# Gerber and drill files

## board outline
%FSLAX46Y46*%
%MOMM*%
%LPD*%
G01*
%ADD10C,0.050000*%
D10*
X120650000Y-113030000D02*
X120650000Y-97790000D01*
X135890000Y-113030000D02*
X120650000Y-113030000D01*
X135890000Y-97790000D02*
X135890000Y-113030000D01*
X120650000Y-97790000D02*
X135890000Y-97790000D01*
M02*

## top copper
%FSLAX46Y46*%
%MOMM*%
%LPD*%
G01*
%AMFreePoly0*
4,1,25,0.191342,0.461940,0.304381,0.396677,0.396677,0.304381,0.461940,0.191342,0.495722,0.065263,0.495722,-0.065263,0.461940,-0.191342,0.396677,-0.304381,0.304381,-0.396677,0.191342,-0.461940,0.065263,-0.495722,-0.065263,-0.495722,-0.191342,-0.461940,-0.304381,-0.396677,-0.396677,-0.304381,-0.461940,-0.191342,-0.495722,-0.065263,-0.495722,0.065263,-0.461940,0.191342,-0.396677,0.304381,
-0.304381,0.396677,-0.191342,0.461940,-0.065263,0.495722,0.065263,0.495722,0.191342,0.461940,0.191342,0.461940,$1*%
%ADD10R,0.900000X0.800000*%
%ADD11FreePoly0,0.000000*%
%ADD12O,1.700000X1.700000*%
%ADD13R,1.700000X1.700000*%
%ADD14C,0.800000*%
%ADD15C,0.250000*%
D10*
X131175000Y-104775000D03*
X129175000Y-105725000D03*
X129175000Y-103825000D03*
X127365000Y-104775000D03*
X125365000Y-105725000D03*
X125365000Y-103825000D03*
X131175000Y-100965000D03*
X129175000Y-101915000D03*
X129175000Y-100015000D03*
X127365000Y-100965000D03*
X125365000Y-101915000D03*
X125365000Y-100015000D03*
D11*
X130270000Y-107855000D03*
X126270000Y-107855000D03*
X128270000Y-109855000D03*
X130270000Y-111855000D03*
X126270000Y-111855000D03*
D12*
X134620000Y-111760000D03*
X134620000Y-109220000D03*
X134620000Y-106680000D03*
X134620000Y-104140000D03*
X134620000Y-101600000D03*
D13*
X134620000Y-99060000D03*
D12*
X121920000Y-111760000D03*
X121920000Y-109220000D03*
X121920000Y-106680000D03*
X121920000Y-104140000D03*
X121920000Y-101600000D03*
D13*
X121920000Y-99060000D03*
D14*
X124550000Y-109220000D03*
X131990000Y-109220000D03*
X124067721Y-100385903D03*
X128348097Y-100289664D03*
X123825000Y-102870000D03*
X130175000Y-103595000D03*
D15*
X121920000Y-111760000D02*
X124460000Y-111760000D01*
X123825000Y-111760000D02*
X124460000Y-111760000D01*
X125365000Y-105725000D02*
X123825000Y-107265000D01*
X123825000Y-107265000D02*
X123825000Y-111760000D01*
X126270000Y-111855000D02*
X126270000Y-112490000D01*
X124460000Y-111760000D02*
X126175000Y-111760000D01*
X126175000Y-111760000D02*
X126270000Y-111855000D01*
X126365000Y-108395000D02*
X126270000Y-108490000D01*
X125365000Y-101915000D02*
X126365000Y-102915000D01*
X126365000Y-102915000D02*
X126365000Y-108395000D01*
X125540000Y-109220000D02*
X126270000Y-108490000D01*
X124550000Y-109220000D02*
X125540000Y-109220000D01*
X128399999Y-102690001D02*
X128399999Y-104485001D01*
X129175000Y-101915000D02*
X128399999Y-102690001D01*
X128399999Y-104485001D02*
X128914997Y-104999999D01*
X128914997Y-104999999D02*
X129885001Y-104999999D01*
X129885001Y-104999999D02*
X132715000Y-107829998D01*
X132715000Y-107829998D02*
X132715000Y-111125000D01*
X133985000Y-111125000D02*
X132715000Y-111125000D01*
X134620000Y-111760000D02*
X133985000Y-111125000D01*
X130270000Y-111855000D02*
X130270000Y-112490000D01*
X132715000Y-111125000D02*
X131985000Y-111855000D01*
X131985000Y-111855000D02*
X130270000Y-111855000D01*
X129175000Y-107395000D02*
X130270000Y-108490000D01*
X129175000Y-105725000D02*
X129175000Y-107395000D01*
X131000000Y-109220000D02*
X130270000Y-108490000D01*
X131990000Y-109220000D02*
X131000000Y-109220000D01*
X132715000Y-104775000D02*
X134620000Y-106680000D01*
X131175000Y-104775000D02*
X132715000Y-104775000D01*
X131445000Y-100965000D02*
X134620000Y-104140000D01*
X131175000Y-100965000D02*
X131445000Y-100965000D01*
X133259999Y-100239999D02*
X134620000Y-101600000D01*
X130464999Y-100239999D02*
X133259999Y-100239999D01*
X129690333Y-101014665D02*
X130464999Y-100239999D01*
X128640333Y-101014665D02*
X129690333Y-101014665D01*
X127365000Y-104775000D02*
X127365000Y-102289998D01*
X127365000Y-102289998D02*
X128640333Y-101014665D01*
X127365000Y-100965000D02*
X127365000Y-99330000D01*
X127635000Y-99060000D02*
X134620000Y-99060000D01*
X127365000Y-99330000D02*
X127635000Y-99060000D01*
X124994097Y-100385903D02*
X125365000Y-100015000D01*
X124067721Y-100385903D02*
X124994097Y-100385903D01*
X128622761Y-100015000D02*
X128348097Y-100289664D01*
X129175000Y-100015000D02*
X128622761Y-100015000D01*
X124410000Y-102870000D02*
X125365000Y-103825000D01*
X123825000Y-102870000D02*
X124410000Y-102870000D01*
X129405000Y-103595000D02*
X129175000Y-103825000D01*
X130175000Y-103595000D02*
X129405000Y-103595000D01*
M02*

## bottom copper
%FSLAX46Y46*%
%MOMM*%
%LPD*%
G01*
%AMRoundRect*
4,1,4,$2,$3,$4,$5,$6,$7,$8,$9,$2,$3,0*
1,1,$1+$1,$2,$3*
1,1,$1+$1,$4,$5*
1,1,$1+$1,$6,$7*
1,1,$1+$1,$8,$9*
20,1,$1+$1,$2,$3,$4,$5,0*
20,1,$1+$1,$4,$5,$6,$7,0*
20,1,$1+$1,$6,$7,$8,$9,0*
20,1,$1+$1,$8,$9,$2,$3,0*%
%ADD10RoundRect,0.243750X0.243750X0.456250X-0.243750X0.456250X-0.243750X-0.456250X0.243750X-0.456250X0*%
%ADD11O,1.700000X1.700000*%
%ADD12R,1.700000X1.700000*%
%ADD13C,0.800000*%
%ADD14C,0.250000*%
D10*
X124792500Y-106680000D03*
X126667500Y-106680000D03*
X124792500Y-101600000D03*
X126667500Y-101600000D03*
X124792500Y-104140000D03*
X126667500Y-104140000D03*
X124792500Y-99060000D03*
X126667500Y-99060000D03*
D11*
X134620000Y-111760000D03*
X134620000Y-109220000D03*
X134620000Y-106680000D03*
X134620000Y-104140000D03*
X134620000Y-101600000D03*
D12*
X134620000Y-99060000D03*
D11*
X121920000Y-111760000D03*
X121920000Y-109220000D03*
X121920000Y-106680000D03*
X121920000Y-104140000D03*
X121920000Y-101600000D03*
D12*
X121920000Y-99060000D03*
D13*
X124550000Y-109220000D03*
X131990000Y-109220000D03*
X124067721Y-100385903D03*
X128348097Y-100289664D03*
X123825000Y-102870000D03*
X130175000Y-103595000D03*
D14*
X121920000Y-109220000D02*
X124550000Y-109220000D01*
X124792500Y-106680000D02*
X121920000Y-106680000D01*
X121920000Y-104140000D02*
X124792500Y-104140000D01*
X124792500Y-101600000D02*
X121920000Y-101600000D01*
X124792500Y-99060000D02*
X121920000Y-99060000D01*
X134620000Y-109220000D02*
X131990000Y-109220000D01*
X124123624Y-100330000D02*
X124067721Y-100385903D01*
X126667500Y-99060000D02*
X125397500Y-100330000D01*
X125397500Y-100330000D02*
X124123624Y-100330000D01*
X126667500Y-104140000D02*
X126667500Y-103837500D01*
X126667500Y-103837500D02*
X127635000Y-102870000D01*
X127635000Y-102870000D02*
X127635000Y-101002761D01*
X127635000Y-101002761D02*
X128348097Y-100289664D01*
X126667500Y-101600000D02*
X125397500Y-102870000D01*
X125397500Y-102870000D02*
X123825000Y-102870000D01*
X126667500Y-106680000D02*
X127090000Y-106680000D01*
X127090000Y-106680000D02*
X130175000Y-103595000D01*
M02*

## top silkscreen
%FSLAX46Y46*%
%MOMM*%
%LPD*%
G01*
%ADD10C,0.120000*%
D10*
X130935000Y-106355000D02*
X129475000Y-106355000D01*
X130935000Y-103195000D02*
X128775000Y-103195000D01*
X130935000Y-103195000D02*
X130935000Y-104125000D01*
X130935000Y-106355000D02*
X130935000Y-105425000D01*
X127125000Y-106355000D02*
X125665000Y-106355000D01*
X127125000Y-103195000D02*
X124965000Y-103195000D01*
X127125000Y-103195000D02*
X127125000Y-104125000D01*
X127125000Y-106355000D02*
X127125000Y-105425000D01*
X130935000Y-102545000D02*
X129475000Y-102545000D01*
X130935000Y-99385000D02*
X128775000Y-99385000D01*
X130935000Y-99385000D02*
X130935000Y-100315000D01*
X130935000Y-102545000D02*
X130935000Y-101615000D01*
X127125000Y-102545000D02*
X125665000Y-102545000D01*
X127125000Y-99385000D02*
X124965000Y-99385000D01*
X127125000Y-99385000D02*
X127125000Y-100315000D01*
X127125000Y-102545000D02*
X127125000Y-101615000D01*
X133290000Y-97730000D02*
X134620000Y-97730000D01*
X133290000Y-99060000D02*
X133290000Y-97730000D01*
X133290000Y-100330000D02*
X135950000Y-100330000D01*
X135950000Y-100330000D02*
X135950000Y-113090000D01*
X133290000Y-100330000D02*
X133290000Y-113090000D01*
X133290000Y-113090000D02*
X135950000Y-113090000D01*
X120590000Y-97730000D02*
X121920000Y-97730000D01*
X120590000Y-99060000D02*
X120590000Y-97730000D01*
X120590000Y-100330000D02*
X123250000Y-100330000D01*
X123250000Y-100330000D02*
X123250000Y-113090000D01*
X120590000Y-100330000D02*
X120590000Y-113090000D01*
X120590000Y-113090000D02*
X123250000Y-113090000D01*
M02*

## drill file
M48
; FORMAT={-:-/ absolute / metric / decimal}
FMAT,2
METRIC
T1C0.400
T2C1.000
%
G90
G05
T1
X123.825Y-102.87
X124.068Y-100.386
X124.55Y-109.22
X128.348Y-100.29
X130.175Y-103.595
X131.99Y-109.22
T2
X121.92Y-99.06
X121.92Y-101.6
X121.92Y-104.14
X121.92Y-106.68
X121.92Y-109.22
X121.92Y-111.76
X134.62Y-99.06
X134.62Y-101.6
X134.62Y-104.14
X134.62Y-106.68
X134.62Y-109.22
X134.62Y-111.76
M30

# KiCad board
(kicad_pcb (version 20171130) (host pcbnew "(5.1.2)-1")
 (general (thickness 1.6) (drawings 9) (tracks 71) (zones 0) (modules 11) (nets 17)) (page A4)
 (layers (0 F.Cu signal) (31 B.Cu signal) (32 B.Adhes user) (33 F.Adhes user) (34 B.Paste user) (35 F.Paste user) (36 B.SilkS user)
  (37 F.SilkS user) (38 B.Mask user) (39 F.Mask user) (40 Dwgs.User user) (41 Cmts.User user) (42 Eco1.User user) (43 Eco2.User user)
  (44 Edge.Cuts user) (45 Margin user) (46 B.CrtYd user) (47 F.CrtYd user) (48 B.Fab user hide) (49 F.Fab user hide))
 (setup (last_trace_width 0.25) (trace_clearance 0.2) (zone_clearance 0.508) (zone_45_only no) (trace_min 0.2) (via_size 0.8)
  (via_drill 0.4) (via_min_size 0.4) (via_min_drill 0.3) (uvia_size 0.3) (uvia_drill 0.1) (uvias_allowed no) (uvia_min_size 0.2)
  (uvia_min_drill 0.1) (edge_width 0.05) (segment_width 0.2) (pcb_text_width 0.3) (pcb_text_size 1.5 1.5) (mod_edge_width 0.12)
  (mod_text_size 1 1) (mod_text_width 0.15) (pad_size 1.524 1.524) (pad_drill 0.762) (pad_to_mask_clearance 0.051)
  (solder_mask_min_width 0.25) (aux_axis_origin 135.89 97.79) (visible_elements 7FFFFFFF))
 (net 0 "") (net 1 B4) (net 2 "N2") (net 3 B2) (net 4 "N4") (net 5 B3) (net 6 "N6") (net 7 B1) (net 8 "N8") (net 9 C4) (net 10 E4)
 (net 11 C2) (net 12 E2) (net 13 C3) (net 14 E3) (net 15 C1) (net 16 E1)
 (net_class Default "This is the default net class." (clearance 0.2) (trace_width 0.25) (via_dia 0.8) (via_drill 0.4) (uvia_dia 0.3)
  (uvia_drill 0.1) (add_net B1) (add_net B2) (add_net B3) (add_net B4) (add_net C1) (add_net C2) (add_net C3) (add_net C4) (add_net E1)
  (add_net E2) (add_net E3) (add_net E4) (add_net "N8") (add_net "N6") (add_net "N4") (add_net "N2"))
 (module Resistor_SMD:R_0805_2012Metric (layer B.Cu) (at 125.73 106.68 180)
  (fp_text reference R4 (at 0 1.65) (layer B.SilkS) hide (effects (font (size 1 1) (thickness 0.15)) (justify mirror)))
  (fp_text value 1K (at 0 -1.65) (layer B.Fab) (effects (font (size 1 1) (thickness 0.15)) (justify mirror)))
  (pad 2 smd roundrect (at 0.9375 0 180) (size 0.975 1.4) (layers B.Cu B.Paste B.Mask) (roundrect_rratio 0.25) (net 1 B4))
  (pad 1 smd roundrect (at -0.9375 0 180) (size 0.975 1.4) (layers B.Cu B.Paste B.Mask) (roundrect_rratio 0.25) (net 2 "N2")))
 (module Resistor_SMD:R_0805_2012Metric (layer B.Cu) (at 125.73 101.6 180)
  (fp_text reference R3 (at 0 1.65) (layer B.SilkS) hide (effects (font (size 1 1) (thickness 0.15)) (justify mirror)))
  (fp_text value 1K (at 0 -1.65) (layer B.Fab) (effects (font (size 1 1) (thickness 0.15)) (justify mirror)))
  (pad 2 smd roundrect (at 0.9375 0 180) (size 0.975 1.4) (layers B.Cu B.Paste B.Mask) (roundrect_rratio 0.25) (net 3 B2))
  (pad 1 smd roundrect (at -0.9375 0 180) (size 0.975 1.4) (layers B.Cu B.Paste B.Mask) (roundrect_rratio 0.25) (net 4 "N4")))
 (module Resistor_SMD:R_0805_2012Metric (layer B.Cu) (at 125.73 104.14 180)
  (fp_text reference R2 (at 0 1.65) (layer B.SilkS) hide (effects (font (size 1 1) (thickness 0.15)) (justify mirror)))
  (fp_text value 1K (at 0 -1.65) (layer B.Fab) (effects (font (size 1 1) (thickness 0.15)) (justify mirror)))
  (pad 2 smd roundrect (at 0.9375 0 180) (size 0.975 1.4) (layers B.Cu B.Paste B.Mask) (roundrect_rratio 0.25) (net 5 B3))
  (pad 1 smd roundrect (at -0.9375 0 180) (size 0.975 1.4) (layers B.Cu B.Paste B.Mask) (roundrect_rratio 0.25) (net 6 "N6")))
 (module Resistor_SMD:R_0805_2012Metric (layer B.Cu) (at 125.73 99.06 180)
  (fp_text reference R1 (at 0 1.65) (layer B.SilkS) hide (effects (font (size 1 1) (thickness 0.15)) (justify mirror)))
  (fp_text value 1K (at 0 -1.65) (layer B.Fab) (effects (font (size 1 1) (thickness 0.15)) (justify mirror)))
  (pad 2 smd roundrect (at 0.9375 0 180) (size 0.975 1.4) (layers B.Cu B.Paste B.Mask) (roundrect_rratio 0.25) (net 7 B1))
  (pad 1 smd roundrect (at -0.9375 0 180) (size 0.975 1.4) (layers B.Cu B.Paste B.Mask) (roundrect_rratio 0.25) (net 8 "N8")))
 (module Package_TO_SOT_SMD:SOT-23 (layer F.Cu) (at 130.175 104.775)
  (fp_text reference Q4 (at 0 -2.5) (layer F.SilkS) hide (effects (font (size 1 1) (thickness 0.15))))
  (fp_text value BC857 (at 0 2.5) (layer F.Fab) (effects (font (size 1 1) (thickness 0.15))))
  (fp_line (start 0.76 1.58) (end -0.7 1.58) (layer F.SilkS) (width 0.12))
  (fp_line (start 0.76 -1.58) (end -1.4 -1.58) (layer F.SilkS) (width 0.12))
  (fp_line (start 0.76 -1.58) (end 0.76 -0.65) (layer F.SilkS) (width 0.12))
  (fp_line (start 0.76 1.58) (end 0.76 0.65) (layer F.SilkS) (width 0.12))
  (pad 3 smd rect (at 1 0) (size 0.9 0.8) (layers F.Cu F.Paste F.Mask) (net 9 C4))
  (pad 2 smd rect (at -1 0.95) (size 0.9 0.8) (layers F.Cu F.Paste F.Mask) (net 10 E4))
  (pad 1 smd rect (at -1 -0.95) (size 0.9 0.8) (layers F.Cu F.Paste F.Mask) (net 2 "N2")))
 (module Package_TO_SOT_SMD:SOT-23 (layer F.Cu) (at 126.365 104.775)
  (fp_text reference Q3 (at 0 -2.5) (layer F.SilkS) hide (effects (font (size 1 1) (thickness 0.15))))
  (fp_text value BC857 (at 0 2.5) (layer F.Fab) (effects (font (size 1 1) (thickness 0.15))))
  (fp_line (start 0.76 1.58) (end -0.7 1.58) (layer F.SilkS) (width 0.12))
  (fp_line (start 0.76 -1.58) (end -1.4 -1.58) (layer F.SilkS) (width 0.12))
  (fp_line (start 0.76 -1.58) (end 0.76 -0.65) (layer F.SilkS) (width 0.12))
  (fp_line (start 0.76 1.58) (end 0.76 0.65) (layer F.SilkS) (width 0.12))
  (pad 3 smd rect (at 1 0) (size 0.9 0.8) (layers F.Cu F.Paste F.Mask) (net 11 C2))
  (pad 2 smd rect (at -1 0.95) (size 0.9 0.8) (layers F.Cu F.Paste F.Mask) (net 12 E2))
  (pad 1 smd rect (at -1 -0.95) (size 0.9 0.8) (layers F.Cu F.Paste F.Mask) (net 4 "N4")))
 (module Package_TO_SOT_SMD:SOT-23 (layer F.Cu) (at 130.175 100.965)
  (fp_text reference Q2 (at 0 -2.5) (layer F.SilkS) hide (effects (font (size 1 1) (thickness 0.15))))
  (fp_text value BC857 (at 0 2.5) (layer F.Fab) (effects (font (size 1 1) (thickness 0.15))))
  (fp_line (start 0.76 1.58) (end -0.7 1.58) (layer F.SilkS) (width 0.12))
  (fp_line (start 0.76 -1.58) (end -1.4 -1.58) (layer F.SilkS) (width 0.12))
  (fp_line (start 0.76 -1.58) (end 0.76 -0.65) (layer F.SilkS) (width 0.12))
  (fp_line (start 0.76 1.58) (end 0.76 0.65) (layer F.SilkS) (width 0.12))
  (pad 3 smd rect (at 1 0) (size 0.9 0.8) (layers F.Cu F.Paste F.Mask) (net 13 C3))
  (pad 2 smd rect (at -1 0.95) (size 0.9 0.8) (layers F.Cu F.Paste F.Mask) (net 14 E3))
  (pad 1 smd rect (at -1 -0.95) (size 0.9 0.8) (layers F.Cu F.Paste F.Mask) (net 6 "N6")))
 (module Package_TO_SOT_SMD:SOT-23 (layer F.Cu) (at 126.365 100.965)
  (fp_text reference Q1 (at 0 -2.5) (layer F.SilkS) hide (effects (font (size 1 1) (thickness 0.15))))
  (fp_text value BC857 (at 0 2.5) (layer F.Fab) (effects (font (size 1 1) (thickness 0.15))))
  (fp_line (start 0.76 1.58) (end -0.7 1.58) (layer F.SilkS) (width 0.12))
  (fp_line (start 0.76 -1.58) (end -1.4 -1.58) (layer F.SilkS) (width 0.12))
  (fp_line (start 0.76 -1.58) (end 0.76 -0.65) (layer F.SilkS) (width 0.12))
  (fp_line (start 0.76 1.58) (end 0.76 0.65) (layer F.SilkS) (width 0.12))
  (pad 3 smd rect (at 1 0) (size 0.9 0.8) (layers F.Cu F.Paste F.Mask) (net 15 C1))
  (pad 2 smd rect (at -1 0.95) (size 0.9 0.8) (layers F.Cu F.Paste F.Mask) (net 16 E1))
  (pad 1 smd rect (at -1 -0.95) (size 0.9 0.8) (layers F.Cu F.Paste F.Mask) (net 8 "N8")))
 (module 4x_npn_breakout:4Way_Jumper (layer F.Cu) (at 128.27 109.855)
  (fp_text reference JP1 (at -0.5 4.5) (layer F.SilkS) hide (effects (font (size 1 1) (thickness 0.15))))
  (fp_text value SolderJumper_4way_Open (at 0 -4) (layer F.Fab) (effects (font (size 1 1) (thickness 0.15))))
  (pad 4 smd custom (at 2 -2) (size 1 1) (layers F.Cu F.Paste F.Mask) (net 10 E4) (options (clearance outline) (anchor circle)) (primitives))
  (pad 1 smd custom (at -2 -2) (size 1 1) (layers F.Cu F.Paste F.Mask) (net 16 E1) (options (clearance outline) (anchor circle))
   (primitives))
  (pad "" smd custom (at 0 0) (size 1 1) (layers F.Cu F.Paste F.Mask) (options (clearance outline) (anchor circle)) (primitives))
  (pad 3 smd custom (at 2 2) (size 1 1) (layers F.Cu F.Paste F.Mask) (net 14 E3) (options (clearance outline) (anchor circle)) (primitives))
  (pad 2 smd custom (at -2 2) (size 1 1) (layers F.Cu F.Paste F.Mask) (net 12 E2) (options (clearance outline) (anchor circle)) (primitives)))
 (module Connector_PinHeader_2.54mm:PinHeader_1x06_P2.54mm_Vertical (layer F.Cu) (at 134.62 99.06)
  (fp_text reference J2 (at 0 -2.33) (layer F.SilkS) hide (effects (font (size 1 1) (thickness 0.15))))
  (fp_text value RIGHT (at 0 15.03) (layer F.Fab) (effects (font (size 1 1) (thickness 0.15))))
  (fp_line (start -1.33 -1.33) (end 0 -1.33) (layer F.SilkS) (width 0.12))
  (fp_line (start -1.33 0) (end -1.33 -1.33) (layer F.SilkS) (width 0.12))
  (fp_line (start -1.33 1.27) (end 1.33 1.27) (layer F.SilkS) (width 0.12))
  (fp_line (start 1.33 1.27) (end 1.33 14.03) (layer F.SilkS) (width 0.12))
  (fp_line (start -1.33 1.27) (end -1.33 14.03) (layer F.SilkS) (width 0.12))
  (fp_line (start -1.33 14.03) (end 1.33 14.03) (layer F.SilkS) (width 0.12))
  (pad 6 thru_hole oval (at 0 12.7) (size 1.7 1.7) (drill 1) (layers *.Cu *.Mask) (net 14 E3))
  (pad 5 thru_hole oval (at 0 10.16) (size 1.7 1.7) (drill 1) (layers *.Cu *.Mask) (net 10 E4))
  (pad 4 thru_hole oval (at 0 7.62) (size 1.7 1.7) (drill 1) (layers *.Cu *.Mask) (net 9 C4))
  (pad 3 thru_hole oval (at 0 5.08) (size 1.7 1.7) (drill 1) (layers *.Cu *.Mask) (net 13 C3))
  (pad 2 thru_hole oval (at 0 2.54) (size 1.7 1.7) (drill 1) (layers *.Cu *.Mask) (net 11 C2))
  (pad 1 thru_hole rect (at 0 0) (size 1.7 1.7) (drill 1) (layers *.Cu *.Mask) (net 15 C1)))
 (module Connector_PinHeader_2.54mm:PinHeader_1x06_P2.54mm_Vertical (layer F.Cu) (at 121.92 99.06)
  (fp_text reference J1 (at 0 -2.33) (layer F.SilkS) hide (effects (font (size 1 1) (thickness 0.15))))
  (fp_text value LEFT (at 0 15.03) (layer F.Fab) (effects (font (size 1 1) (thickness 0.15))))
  (fp_line (start -1.33 -1.33) (end 0 -1.33) (layer F.SilkS) (width 0.12))
  (fp_line (start -1.33 0) (end -1.33 -1.33) (layer F.SilkS) (width 0.12))
  (fp_line (start -1.33 1.27) (end 1.33 1.27) (layer F.SilkS) (width 0.12))
  (fp_line (start 1.33 1.27) (end 1.33 14.03) (layer F.SilkS) (width 0.12))
  (fp_line (start -1.33 1.27) (end -1.33 14.03) (layer F.SilkS) (width 0.12))
  (fp_line (start -1.33 14.03) (end 1.33 14.03) (layer F.SilkS) (width 0.12))
  (pad 6 thru_hole oval (at 0 12.7) (size 1.7 1.7) (drill 1) (layers *.Cu *.Mask) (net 12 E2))
  (pad 5 thru_hole oval (at 0 10.16) (size 1.7 1.7) (drill 1) (layers *.Cu *.Mask) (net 16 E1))
  (pad 4 thru_hole oval (at 0 7.62) (size 1.7 1.7) (drill 1) (layers *.Cu *.Mask) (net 1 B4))
  (pad 3 thru_hole oval (at 0 5.08) (size 1.7 1.7) (drill 1) (layers *.Cu *.Mask) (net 5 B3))
  (pad 2 thru_hole oval (at 0 2.54) (size 1.7 1.7) (drill 1) (layers *.Cu *.Mask) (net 3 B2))
  (pad 1 thru_hole rect (at 0 0) (size 1.7 1.7) (drill 1) (layers *.Cu *.Mask) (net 7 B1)))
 (gr_line (start 120.65 113.03) (end 120.65 97.79) (layer Edge.Cuts) (width 0.05))
 (gr_line (start 135.89 113.03) (end 120.65 113.03) (layer Edge.Cuts) (width 0.05))
 (gr_line (start 135.89 97.79) (end 135.89 113.03) (layer Edge.Cuts) (width 0.05))
 (gr_line (start 120.65 97.79) (end 135.89 97.79) (layer Edge.Cuts) (width 0.05))
 (segment (start 121.92 111.76) (end 124.46 111.76) (width 0.25) (layer F.Cu) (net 12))
 (segment (start 123.825 111.76) (end 124.46 111.76) (width 0.25) (layer F.Cu) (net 12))
 (segment (start 125.365 105.725) (end 123.825 107.265) (width 0.25) (layer F.Cu) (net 12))
 (segment (start 123.825 107.265) (end 123.825 111.76) (width 0.25) (layer F.Cu) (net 12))
 (segment (start 126.27 111.855) (end 126.27 112.49) (width 0.25) (layer F.Cu) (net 12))
 (segment (start 124.46 111.76) (end 126.175 111.76) (width 0.25) (layer F.Cu) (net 12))
 (segment (start 126.175 111.76) (end 126.27 111.855) (width 0.25) (layer F.Cu) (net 12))
 (segment (start 126.365 108.395) (end 126.27 108.49) (width 0.25) (layer F.Cu) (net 16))
 (segment (start 125.365 101.915) (end 126.365 102.915) (width 0.25) (layer F.Cu) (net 16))
 (segment (start 126.365 102.915) (end 126.365 108.395) (width 0.25) (layer F.Cu) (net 16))
 (via (at 124.55 109.22) (size 0.8) (drill 0.4) (layers F.Cu B.Cu) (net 16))
 (segment (start 121.92 109.22) (end 124.55 109.22) (width 0.25) (layer B.Cu) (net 16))
 (segment (start 125.54 109.22) (end 126.27 108.49) (width 0.25) (layer F.Cu) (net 16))
 (segment (start 124.55 109.22) (end 125.54 109.22) (width 0.25) (layer F.Cu) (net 16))
 (segment (start 124.7925 106.68) (end 121.92 106.68) (width 0.25) (layer B.Cu) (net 1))
 (segment (start 121.92 104.14) (end 124.7925 104.14) (width 0.25) (layer B.Cu) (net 5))
 (segment (start 124.7925 101.6) (end 121.92 101.6) (width 0.25) (layer B.Cu) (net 3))
 (segment (start 124.7925 99.06) (end 121.92 99.06) (width 0.25) (layer B.Cu) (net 7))
 (segment (start 128.399999 102.690001) (end 128.399999 104.485001) (width 0.25) (layer F.Cu) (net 14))
 (segment (start 129.175 101.915) (end 128.399999 102.690001) (width 0.25) (layer F.Cu) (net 14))
 (segment (start 128.399999 104.485001) (end 128.914997 104.999999) (width 0.25) (layer F.Cu) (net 14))
 (segment (start 128.914997 104.999999) (end 129.885001 104.999999) (width 0.25) (layer F.Cu) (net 14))
 (segment (start 129.885001 104.999999) (end 132.715 107.829998) (width 0.25) (layer F.Cu) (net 14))
 (segment (start 132.715 107.829998) (end 132.715 111.125) (width 0.25) (layer F.Cu) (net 14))
 (segment (start 133.985 111.125) (end 132.715 111.125) (width 0.25) (layer F.Cu) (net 14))
 (segment (start 134.62 111.76) (end 133.985 111.125) (width 0.25) (layer F.Cu) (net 14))
 (segment (start 130.27 111.855) (end 130.27 112.49) (width 0.25) (layer F.Cu) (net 14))
 (segment (start 132.715 111.125) (end 131.985 111.855) (width 0.25) (layer F.Cu) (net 14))
 (segment (start 131.985 111.855) (end 130.27 111.855) (width 0.25) (layer F.Cu) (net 14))
 (segment (start 129.175 107.395) (end 130.27 108.49) (width 0.25) (layer F.Cu) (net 10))
 (segment (start 129.175 105.725) (end 129.175 107.395) (width 0.25) (layer F.Cu) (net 10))
 (via (at 131.99 109.22) (size 0.8) (drill 0.4) (layers F.Cu B.Cu) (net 10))
 (segment (start 134.62 109.22) (end 131.99 109.22) (width 0.25) (layer B.Cu) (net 10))
 (segment (start 131 109.22) (end 130.27 108.49) (width 0.25) (layer F.Cu) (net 10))
 (segment (start 131.99 109.22) (end 131 109.22) (width 0.25) (layer F.Cu) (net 10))
 (segment (start 132.715 104.775) (end 134.62 106.68) (width 0.25) (layer F.Cu) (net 9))
 (segment (start 131.175 104.775) (end 132.715 104.775) (width 0.25) (layer F.Cu) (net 9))
 (segment (start 131.445 100.965) (end 134.62 104.14) (width 0.25) (layer F.Cu) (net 13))
 (segment (start 131.175 100.965) (end 131.445 100.965) (width 0.25) (layer F.Cu) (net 13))
 (segment (start 133.259999 100.239999) (end 134.62 101.6) (width 0.25) (layer F.Cu) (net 11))
 (segment (start 130.464999 100.239999) (end 133.259999 100.239999) (width 0.25) (layer F.Cu) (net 11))
 (segment (start 129.690333 101.014665) (end 130.464999 100.239999) (width 0.25) (layer F.Cu) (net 11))
 (segment (start 128.640333 101.014665) (end 129.690333 101.014665) (width 0.25) (layer F.Cu) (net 11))
 (segment (start 127.365 104.775) (end 127.365 102.289998) (width 0.25) (layer F.Cu) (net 11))
 (segment (start 127.365 102.289998) (end 128.640333 101.014665) (width 0.25) (layer F.Cu) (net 11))
 (segment (start 127.365 100.965) (end 127.365 99.33) (width 0.25) (layer F.Cu) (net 15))
 (segment (start 127.635 99.06) (end 134.62 99.06) (width 0.25) (layer F.Cu) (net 15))
 (segment (start 127.365 99.33) (end 127.635 99.06) (width 0.25) (layer F.Cu) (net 15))
 (via (at 124.067721 100.385903) (size 0.8) (drill 0.4) (layers F.Cu B.Cu) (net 8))
 (segment (start 124.994097 100.385903) (end 125.365 100.015) (width 0.25) (layer F.Cu) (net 8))
 (segment (start 124.067721 100.385903) (end 124.994097 100.385903) (width 0.25) (layer F.Cu) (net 8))
 (segment (start 124.123624 100.33) (end 124.067721 100.385903) (width 0.25) (layer B.Cu) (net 8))
 (segment (start 126.6675 99.06) (end 125.3975 100.33) (width 0.25) (layer B.Cu) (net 8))
 (segment (start 125.3975 100.33) (end 124.123624 100.33) (width 0.25) (layer B.Cu) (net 8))
 (segment (start 126.6675 104.14) (end 126.6675 103.8375) (width 0.25) (layer B.Cu) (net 6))
 (segment (start 126.6675 103.8375) (end 127.635 102.87) (width 0.25) (layer B.Cu) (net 6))
 (via (at 128.348097 100.289664) (size 0.8) (drill 0.4) (layers F.Cu B.Cu) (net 6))
 (segment (start 127.635 102.87) (end 127.635 101.002761) (width 0.25) (layer B.Cu) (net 6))
 (segment (start 127.635 101.002761) (end 128.348097 100.289664) (width 0.25) (layer B.Cu) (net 6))
 (segment (start 128.622761 100.015) (end 128.348097 100.289664) (width 0.25) (layer F.Cu) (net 6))
 (segment (start 129.175 100.015) (end 128.622761 100.015) (width 0.25) (layer F.Cu) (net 6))
 (via (at 123.825 102.87) (size 0.8) (drill 0.4) (layers F.Cu B.Cu) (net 4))
 (segment (start 126.6675 101.6) (end 125.3975 102.87) (width 0.25) (layer B.Cu) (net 4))
 (segment (start 125.3975 102.87) (end 123.825 102.87) (width 0.25) (layer B.Cu) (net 4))
 (segment (start 124.41 102.87) (end 125.365 103.825) (width 0.25) (layer F.Cu) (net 4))
 (segment (start 123.825 102.87) (end 124.41 102.87) (width 0.25) (layer F.Cu) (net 4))
 (via (at 130.175 103.595) (size 0.8) (drill 0.4) (layers F.Cu B.Cu) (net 2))
 (segment (start 126.6675 106.68) (end 127.09 106.68) (width 0.25) (layer B.Cu) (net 2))
 (segment (start 127.09 106.68) (end 130.175 103.595) (width 0.25) (layer B.Cu) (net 2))
 (segment (start 129.405 103.595) (end 129.175 103.825) (width 0.25) (layer F.Cu) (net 2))
 (segment (start 130.175 103.595) (end 129.405 103.595) (width 0.25) (layer F.Cu) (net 2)))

